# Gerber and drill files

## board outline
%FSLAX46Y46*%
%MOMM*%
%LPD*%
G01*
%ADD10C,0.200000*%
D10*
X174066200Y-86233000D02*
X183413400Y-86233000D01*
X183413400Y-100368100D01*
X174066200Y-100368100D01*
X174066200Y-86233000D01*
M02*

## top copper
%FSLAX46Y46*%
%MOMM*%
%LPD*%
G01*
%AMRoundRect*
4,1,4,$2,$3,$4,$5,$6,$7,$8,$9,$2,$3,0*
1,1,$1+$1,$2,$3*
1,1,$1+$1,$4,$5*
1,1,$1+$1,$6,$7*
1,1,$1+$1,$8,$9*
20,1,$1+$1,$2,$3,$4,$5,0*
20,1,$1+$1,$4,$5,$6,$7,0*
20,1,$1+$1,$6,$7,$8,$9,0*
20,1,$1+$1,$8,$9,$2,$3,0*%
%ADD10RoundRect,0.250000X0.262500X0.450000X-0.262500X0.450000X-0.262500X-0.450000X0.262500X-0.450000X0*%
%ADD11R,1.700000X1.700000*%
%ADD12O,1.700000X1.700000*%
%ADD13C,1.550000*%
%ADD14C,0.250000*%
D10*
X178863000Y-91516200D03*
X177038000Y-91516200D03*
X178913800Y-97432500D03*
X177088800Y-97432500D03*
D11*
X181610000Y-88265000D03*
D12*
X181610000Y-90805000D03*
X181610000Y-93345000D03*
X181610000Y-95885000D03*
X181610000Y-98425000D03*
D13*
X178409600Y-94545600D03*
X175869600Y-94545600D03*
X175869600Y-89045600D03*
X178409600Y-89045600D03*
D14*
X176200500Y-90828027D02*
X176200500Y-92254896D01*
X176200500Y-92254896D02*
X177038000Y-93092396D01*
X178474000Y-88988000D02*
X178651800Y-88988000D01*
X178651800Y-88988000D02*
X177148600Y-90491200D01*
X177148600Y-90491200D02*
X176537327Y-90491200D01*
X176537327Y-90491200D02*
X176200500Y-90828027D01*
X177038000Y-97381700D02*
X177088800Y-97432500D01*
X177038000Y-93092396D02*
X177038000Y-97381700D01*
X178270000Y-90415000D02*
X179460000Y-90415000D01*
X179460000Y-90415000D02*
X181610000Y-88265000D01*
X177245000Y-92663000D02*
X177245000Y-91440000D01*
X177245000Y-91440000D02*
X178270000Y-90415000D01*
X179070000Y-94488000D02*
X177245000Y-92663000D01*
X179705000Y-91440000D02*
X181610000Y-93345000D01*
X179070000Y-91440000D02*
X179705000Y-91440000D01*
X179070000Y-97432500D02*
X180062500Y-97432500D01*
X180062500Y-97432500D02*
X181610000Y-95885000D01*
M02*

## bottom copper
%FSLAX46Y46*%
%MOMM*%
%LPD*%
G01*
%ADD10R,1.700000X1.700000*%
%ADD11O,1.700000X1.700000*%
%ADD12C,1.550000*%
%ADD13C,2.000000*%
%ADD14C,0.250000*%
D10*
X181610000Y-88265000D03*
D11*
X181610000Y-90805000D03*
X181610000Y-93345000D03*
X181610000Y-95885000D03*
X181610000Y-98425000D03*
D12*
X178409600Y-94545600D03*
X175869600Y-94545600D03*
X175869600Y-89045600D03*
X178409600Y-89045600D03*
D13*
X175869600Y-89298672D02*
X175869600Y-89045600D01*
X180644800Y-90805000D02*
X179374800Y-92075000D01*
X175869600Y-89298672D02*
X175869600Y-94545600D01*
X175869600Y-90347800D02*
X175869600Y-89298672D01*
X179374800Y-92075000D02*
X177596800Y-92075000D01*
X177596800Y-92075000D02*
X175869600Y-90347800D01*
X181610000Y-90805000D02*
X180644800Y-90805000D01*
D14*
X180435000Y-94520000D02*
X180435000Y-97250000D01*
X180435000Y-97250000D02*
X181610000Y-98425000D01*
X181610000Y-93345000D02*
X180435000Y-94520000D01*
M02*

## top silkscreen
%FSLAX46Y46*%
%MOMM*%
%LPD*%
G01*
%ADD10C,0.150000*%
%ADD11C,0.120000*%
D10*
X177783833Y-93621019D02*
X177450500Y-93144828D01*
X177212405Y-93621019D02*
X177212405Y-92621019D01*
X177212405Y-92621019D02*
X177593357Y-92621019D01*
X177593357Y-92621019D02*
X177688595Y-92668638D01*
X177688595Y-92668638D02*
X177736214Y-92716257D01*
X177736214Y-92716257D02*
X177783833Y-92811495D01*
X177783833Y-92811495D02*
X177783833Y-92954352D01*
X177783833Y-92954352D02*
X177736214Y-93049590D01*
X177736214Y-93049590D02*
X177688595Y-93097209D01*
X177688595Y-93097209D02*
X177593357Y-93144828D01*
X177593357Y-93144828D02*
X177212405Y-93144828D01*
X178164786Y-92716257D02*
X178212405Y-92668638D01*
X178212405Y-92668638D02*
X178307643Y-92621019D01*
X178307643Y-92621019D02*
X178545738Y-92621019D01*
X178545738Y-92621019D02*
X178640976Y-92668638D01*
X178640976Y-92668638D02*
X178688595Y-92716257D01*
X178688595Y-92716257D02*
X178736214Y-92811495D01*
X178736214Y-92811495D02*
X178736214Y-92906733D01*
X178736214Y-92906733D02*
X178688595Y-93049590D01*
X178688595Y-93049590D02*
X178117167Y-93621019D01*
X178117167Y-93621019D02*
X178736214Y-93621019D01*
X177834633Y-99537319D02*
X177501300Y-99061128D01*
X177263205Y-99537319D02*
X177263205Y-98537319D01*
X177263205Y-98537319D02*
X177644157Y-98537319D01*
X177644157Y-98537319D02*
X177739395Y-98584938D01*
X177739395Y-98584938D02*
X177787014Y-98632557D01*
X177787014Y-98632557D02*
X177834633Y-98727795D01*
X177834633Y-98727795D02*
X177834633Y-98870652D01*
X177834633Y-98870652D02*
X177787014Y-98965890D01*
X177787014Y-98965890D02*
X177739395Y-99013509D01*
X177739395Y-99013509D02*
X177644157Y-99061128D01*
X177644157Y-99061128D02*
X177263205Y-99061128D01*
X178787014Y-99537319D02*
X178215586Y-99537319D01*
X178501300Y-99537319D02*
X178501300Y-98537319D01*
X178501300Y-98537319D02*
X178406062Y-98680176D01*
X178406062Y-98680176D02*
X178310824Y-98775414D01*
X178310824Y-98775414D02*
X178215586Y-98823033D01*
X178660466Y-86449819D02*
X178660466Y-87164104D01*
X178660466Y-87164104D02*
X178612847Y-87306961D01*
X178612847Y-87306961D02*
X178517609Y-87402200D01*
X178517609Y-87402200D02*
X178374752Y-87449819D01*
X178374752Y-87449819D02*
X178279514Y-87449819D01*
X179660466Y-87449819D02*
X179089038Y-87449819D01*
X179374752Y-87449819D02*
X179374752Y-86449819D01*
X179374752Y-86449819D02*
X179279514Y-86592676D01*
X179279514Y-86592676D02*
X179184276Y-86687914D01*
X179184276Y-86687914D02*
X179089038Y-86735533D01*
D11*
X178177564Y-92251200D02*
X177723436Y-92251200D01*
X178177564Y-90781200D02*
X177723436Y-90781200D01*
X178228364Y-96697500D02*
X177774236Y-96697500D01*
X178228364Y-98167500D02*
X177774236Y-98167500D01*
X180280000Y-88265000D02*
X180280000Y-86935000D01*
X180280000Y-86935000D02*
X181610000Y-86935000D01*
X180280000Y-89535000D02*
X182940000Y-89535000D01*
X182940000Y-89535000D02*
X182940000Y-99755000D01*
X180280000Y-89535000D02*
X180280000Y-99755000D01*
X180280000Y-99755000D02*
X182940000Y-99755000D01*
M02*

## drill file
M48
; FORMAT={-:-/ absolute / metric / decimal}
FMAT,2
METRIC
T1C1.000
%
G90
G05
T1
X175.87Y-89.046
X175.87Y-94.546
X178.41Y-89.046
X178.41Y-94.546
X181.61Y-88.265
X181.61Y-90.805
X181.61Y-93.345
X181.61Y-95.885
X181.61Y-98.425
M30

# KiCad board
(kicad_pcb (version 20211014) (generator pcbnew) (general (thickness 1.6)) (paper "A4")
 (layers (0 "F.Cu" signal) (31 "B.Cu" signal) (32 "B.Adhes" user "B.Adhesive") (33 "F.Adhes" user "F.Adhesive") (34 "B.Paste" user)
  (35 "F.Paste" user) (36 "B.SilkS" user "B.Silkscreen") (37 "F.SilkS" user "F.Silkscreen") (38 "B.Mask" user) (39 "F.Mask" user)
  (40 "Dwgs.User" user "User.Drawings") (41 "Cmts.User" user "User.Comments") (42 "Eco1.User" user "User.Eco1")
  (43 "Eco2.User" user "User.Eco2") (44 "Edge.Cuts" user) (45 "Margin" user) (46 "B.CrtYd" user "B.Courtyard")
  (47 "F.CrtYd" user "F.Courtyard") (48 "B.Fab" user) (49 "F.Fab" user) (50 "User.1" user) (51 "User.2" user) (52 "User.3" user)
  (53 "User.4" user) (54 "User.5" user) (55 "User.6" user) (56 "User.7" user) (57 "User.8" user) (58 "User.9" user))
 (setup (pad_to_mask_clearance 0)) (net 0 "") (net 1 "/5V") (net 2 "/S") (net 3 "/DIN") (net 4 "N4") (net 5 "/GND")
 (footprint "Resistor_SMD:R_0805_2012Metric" (layer "F.Cu") (at 177.9505 91.5162 180)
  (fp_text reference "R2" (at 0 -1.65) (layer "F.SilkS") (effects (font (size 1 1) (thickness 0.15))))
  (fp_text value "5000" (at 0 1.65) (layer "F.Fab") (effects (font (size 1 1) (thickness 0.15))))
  (fp_line (start -0.227064 -0.735) (end 0.227064 -0.735) (layer "F.SilkS") (width 0.12))
  (fp_line (start -0.227064 0.735) (end 0.227064 0.735) (layer "F.SilkS") (width 0.12))
  (pad "1" smd roundrect (at -0.9125 0 180) (size 1.025 1.4) (layers "F.Cu" "F.Paste" "F.Mask") (roundrect_rratio 0.243902) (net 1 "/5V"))
  (pad "2" smd roundrect (at 0.9125 0 180) (size 1.025 1.4) (layers "F.Cu" "F.Paste" "F.Mask") (roundrect_rratio 0.243902) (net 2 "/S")))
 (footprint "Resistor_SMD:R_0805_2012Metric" (layer "F.Cu") (at 178.0013 97.4325 180)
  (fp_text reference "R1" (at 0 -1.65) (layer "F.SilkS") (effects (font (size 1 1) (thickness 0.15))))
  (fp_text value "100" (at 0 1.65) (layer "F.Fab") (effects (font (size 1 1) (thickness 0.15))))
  (fp_line (start -0.227064 0.735) (end 0.227064 0.735) (layer "F.SilkS") (width 0.12))
  (fp_line (start -0.227064 -0.735) (end 0.227064 -0.735) (layer "F.SilkS") (width 0.12))
  (pad "1" smd roundrect (at -0.9125 0 180) (size 1.025 1.4) (layers "F.Cu" "F.Paste" "F.Mask") (roundrect_rratio 0.243902) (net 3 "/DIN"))
  (pad "2" smd roundrect (at 0.9125 0 180) (size 1.025 1.4) (layers "F.Cu" "F.Paste" "F.Mask") (roundrect_rratio 0.243902) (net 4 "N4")))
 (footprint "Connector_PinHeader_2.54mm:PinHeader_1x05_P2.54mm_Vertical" (layer "F.Cu") (at 181.61 88.265)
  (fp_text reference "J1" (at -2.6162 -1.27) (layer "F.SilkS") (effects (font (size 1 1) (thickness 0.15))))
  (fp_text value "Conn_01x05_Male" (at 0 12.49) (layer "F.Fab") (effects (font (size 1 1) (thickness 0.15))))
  (fp_line (start -1.33 0) (end -1.33 -1.33) (layer "F.SilkS") (width 0.12))
  (fp_line (start -1.33 -1.33) (end 0 -1.33) (layer "F.SilkS") (width 0.12))
  (fp_line (start -1.33 1.27) (end 1.33 1.27) (layer "F.SilkS") (width 0.12))
  (fp_line (start 1.33 1.27) (end 1.33 11.49) (layer "F.SilkS") (width 0.12))
  (fp_line (start -1.33 1.27) (end -1.33 11.49) (layer "F.SilkS") (width 0.12))
  (fp_line (start -1.33 11.49) (end 1.33 11.49) (layer "F.SilkS") (width 0.12))
  (pad "1" thru_hole rect (at 0 0) (size 1.7 1.7) (drill 1) (layers *.Cu *.Mask) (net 2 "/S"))
  (pad "2" thru_hole oval (at 0 2.54) (size 1.7 1.7) (drill 1) (layers *.Cu *.Mask) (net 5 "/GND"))
  (pad "3" thru_hole oval (at 0 5.08) (size 1.7 1.7) (drill 1) (layers *.Cu *.Mask) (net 1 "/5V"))
  (pad "4" thru_hole oval (at 0 7.62) (size 1.7 1.7) (drill 1) (layers *.Cu *.Mask) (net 3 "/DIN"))
  (pad "5" thru_hole oval (at 0 10.16) (size 1.7 1.7) (drill 1) (layers *.Cu *.Mask) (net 1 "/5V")))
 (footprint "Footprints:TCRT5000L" (layer "B.Cu") (at 177.1396 91.7956 90)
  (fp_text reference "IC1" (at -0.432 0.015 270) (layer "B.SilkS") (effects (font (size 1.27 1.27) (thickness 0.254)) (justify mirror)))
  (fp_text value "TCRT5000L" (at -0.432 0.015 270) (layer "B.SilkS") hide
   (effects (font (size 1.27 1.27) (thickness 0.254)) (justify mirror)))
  (pad "1" thru_hole circle locked (at -2.75 1.27 90) (size 1.55 1.55) (drill 1) (layers *.Cu *.Mask) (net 2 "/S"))
  (pad "2" thru_hole circle locked (at -2.75 -1.27 90) (size 1.55 1.55) (drill 1) (layers *.Cu *.Mask) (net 5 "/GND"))
  (pad "3" thru_hole circle locked (at 2.75 -1.27 90) (size 1.55 1.55) (drill 1) (layers *.Cu *.Mask) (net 5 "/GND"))
  (pad "4" thru_hole circle locked (at 2.75 1.27 90) (size 1.55 1.55) (drill 1) (layers *.Cu *.Mask) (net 4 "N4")))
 (gr_rect (start 174.0662 86.233) (end 183.4134 100.3681) (layer "Edge.Cuts") (width 0.2) (fill none))
 (segment (start 176.2005 90.828027) (end 176.2005 92.254896) (width 0.25) (layer "F.Cu") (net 4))
 (segment (start 176.2005 92.254896) (end 177.038 93.092396) (width 0.25) (layer "F.Cu") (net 4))
 (segment (start 178.474 88.988) (end 178.6518 88.988) (width 0.25) (layer "F.Cu") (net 4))
 (segment (start 178.6518 88.988) (end 177.1486 90.4912) (width 0.25) (layer "F.Cu") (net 4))
 (segment (start 177.1486 90.4912) (end 176.537327 90.4912) (width 0.25) (layer "F.Cu") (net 4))
 (segment (start 176.537327 90.4912) (end 176.2005 90.828027) (width 0.25) (layer "F.Cu") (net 4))
 (segment (start 177.038 97.3817) (end 177.0888 97.4325) (width 0.25) (layer "F.Cu") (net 4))
 (segment (start 177.038 93.092396) (end 177.038 97.3817) (width 0.25) (layer "F.Cu") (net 4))
 (segment (start 178.27 90.415) (end 179.46 90.415) (width 0.25) (layer "F.Cu") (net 2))
 (segment (start 179.46 90.415) (end 181.61 88.265) (width 0.25) (layer "F.Cu") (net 2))
 (segment (start 177.245 92.663) (end 177.245 91.44) (width 0.25) (layer "F.Cu") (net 2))
 (segment (start 177.245 91.44) (end 178.27 90.415) (width 0.25) (layer "F.Cu") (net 2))
 (segment (start 179.07 94.488) (end 177.245 92.663) (width 0.25) (layer "F.Cu") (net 2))
 (segment (start 175.8696 89.298672) (end 175.8696 89.0456) (width 2) (layer "B.Cu") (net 5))
 (segment (start 180.6448 90.805) (end 179.3748 92.075) (width 2) (layer "B.Cu") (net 5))
 (segment (start 175.8696 89.298672) (end 175.8696 94.5456) (width 2) (layer "B.Cu") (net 5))
 (segment (start 175.8696 90.3478) (end 175.8696 89.298672) (width 2) (layer "B.Cu") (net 5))
 (segment (start 179.3748 92.075) (end 177.5968 92.075) (width 2) (layer "B.Cu") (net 5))
 (segment (start 177.5968 92.075) (end 175.8696 90.3478) (width 2) (layer "B.Cu") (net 5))
 (segment (start 181.61 90.805) (end 180.6448 90.805) (width 2) (layer "B.Cu") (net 5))
 (segment (start 179.705 91.44) (end 181.61 93.345) (width 0.25) (layer "F.Cu") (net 1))
 (segment (start 179.07 91.44) (end 179.705 91.44) (width 0.25) (layer "F.Cu") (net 1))
 (segment (start 180.435 94.52) (end 180.435 97.25) (width 0.25) (layer "B.Cu") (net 1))
 (segment (start 180.435 97.25) (end 181.61 98.425) (width 0.25) (layer "B.Cu") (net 1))
 (segment (start 181.61 93.345) (end 180.435 94.52) (width 0.25) (layer "B.Cu") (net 1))
 (segment (start 179.07 97.4325) (end 180.0625 97.4325) (width 0.25) (layer "F.Cu") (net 3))
 (segment (start 180.0625 97.4325) (end 181.61 95.885) (width 0.25) (layer "F.Cu") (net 3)))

